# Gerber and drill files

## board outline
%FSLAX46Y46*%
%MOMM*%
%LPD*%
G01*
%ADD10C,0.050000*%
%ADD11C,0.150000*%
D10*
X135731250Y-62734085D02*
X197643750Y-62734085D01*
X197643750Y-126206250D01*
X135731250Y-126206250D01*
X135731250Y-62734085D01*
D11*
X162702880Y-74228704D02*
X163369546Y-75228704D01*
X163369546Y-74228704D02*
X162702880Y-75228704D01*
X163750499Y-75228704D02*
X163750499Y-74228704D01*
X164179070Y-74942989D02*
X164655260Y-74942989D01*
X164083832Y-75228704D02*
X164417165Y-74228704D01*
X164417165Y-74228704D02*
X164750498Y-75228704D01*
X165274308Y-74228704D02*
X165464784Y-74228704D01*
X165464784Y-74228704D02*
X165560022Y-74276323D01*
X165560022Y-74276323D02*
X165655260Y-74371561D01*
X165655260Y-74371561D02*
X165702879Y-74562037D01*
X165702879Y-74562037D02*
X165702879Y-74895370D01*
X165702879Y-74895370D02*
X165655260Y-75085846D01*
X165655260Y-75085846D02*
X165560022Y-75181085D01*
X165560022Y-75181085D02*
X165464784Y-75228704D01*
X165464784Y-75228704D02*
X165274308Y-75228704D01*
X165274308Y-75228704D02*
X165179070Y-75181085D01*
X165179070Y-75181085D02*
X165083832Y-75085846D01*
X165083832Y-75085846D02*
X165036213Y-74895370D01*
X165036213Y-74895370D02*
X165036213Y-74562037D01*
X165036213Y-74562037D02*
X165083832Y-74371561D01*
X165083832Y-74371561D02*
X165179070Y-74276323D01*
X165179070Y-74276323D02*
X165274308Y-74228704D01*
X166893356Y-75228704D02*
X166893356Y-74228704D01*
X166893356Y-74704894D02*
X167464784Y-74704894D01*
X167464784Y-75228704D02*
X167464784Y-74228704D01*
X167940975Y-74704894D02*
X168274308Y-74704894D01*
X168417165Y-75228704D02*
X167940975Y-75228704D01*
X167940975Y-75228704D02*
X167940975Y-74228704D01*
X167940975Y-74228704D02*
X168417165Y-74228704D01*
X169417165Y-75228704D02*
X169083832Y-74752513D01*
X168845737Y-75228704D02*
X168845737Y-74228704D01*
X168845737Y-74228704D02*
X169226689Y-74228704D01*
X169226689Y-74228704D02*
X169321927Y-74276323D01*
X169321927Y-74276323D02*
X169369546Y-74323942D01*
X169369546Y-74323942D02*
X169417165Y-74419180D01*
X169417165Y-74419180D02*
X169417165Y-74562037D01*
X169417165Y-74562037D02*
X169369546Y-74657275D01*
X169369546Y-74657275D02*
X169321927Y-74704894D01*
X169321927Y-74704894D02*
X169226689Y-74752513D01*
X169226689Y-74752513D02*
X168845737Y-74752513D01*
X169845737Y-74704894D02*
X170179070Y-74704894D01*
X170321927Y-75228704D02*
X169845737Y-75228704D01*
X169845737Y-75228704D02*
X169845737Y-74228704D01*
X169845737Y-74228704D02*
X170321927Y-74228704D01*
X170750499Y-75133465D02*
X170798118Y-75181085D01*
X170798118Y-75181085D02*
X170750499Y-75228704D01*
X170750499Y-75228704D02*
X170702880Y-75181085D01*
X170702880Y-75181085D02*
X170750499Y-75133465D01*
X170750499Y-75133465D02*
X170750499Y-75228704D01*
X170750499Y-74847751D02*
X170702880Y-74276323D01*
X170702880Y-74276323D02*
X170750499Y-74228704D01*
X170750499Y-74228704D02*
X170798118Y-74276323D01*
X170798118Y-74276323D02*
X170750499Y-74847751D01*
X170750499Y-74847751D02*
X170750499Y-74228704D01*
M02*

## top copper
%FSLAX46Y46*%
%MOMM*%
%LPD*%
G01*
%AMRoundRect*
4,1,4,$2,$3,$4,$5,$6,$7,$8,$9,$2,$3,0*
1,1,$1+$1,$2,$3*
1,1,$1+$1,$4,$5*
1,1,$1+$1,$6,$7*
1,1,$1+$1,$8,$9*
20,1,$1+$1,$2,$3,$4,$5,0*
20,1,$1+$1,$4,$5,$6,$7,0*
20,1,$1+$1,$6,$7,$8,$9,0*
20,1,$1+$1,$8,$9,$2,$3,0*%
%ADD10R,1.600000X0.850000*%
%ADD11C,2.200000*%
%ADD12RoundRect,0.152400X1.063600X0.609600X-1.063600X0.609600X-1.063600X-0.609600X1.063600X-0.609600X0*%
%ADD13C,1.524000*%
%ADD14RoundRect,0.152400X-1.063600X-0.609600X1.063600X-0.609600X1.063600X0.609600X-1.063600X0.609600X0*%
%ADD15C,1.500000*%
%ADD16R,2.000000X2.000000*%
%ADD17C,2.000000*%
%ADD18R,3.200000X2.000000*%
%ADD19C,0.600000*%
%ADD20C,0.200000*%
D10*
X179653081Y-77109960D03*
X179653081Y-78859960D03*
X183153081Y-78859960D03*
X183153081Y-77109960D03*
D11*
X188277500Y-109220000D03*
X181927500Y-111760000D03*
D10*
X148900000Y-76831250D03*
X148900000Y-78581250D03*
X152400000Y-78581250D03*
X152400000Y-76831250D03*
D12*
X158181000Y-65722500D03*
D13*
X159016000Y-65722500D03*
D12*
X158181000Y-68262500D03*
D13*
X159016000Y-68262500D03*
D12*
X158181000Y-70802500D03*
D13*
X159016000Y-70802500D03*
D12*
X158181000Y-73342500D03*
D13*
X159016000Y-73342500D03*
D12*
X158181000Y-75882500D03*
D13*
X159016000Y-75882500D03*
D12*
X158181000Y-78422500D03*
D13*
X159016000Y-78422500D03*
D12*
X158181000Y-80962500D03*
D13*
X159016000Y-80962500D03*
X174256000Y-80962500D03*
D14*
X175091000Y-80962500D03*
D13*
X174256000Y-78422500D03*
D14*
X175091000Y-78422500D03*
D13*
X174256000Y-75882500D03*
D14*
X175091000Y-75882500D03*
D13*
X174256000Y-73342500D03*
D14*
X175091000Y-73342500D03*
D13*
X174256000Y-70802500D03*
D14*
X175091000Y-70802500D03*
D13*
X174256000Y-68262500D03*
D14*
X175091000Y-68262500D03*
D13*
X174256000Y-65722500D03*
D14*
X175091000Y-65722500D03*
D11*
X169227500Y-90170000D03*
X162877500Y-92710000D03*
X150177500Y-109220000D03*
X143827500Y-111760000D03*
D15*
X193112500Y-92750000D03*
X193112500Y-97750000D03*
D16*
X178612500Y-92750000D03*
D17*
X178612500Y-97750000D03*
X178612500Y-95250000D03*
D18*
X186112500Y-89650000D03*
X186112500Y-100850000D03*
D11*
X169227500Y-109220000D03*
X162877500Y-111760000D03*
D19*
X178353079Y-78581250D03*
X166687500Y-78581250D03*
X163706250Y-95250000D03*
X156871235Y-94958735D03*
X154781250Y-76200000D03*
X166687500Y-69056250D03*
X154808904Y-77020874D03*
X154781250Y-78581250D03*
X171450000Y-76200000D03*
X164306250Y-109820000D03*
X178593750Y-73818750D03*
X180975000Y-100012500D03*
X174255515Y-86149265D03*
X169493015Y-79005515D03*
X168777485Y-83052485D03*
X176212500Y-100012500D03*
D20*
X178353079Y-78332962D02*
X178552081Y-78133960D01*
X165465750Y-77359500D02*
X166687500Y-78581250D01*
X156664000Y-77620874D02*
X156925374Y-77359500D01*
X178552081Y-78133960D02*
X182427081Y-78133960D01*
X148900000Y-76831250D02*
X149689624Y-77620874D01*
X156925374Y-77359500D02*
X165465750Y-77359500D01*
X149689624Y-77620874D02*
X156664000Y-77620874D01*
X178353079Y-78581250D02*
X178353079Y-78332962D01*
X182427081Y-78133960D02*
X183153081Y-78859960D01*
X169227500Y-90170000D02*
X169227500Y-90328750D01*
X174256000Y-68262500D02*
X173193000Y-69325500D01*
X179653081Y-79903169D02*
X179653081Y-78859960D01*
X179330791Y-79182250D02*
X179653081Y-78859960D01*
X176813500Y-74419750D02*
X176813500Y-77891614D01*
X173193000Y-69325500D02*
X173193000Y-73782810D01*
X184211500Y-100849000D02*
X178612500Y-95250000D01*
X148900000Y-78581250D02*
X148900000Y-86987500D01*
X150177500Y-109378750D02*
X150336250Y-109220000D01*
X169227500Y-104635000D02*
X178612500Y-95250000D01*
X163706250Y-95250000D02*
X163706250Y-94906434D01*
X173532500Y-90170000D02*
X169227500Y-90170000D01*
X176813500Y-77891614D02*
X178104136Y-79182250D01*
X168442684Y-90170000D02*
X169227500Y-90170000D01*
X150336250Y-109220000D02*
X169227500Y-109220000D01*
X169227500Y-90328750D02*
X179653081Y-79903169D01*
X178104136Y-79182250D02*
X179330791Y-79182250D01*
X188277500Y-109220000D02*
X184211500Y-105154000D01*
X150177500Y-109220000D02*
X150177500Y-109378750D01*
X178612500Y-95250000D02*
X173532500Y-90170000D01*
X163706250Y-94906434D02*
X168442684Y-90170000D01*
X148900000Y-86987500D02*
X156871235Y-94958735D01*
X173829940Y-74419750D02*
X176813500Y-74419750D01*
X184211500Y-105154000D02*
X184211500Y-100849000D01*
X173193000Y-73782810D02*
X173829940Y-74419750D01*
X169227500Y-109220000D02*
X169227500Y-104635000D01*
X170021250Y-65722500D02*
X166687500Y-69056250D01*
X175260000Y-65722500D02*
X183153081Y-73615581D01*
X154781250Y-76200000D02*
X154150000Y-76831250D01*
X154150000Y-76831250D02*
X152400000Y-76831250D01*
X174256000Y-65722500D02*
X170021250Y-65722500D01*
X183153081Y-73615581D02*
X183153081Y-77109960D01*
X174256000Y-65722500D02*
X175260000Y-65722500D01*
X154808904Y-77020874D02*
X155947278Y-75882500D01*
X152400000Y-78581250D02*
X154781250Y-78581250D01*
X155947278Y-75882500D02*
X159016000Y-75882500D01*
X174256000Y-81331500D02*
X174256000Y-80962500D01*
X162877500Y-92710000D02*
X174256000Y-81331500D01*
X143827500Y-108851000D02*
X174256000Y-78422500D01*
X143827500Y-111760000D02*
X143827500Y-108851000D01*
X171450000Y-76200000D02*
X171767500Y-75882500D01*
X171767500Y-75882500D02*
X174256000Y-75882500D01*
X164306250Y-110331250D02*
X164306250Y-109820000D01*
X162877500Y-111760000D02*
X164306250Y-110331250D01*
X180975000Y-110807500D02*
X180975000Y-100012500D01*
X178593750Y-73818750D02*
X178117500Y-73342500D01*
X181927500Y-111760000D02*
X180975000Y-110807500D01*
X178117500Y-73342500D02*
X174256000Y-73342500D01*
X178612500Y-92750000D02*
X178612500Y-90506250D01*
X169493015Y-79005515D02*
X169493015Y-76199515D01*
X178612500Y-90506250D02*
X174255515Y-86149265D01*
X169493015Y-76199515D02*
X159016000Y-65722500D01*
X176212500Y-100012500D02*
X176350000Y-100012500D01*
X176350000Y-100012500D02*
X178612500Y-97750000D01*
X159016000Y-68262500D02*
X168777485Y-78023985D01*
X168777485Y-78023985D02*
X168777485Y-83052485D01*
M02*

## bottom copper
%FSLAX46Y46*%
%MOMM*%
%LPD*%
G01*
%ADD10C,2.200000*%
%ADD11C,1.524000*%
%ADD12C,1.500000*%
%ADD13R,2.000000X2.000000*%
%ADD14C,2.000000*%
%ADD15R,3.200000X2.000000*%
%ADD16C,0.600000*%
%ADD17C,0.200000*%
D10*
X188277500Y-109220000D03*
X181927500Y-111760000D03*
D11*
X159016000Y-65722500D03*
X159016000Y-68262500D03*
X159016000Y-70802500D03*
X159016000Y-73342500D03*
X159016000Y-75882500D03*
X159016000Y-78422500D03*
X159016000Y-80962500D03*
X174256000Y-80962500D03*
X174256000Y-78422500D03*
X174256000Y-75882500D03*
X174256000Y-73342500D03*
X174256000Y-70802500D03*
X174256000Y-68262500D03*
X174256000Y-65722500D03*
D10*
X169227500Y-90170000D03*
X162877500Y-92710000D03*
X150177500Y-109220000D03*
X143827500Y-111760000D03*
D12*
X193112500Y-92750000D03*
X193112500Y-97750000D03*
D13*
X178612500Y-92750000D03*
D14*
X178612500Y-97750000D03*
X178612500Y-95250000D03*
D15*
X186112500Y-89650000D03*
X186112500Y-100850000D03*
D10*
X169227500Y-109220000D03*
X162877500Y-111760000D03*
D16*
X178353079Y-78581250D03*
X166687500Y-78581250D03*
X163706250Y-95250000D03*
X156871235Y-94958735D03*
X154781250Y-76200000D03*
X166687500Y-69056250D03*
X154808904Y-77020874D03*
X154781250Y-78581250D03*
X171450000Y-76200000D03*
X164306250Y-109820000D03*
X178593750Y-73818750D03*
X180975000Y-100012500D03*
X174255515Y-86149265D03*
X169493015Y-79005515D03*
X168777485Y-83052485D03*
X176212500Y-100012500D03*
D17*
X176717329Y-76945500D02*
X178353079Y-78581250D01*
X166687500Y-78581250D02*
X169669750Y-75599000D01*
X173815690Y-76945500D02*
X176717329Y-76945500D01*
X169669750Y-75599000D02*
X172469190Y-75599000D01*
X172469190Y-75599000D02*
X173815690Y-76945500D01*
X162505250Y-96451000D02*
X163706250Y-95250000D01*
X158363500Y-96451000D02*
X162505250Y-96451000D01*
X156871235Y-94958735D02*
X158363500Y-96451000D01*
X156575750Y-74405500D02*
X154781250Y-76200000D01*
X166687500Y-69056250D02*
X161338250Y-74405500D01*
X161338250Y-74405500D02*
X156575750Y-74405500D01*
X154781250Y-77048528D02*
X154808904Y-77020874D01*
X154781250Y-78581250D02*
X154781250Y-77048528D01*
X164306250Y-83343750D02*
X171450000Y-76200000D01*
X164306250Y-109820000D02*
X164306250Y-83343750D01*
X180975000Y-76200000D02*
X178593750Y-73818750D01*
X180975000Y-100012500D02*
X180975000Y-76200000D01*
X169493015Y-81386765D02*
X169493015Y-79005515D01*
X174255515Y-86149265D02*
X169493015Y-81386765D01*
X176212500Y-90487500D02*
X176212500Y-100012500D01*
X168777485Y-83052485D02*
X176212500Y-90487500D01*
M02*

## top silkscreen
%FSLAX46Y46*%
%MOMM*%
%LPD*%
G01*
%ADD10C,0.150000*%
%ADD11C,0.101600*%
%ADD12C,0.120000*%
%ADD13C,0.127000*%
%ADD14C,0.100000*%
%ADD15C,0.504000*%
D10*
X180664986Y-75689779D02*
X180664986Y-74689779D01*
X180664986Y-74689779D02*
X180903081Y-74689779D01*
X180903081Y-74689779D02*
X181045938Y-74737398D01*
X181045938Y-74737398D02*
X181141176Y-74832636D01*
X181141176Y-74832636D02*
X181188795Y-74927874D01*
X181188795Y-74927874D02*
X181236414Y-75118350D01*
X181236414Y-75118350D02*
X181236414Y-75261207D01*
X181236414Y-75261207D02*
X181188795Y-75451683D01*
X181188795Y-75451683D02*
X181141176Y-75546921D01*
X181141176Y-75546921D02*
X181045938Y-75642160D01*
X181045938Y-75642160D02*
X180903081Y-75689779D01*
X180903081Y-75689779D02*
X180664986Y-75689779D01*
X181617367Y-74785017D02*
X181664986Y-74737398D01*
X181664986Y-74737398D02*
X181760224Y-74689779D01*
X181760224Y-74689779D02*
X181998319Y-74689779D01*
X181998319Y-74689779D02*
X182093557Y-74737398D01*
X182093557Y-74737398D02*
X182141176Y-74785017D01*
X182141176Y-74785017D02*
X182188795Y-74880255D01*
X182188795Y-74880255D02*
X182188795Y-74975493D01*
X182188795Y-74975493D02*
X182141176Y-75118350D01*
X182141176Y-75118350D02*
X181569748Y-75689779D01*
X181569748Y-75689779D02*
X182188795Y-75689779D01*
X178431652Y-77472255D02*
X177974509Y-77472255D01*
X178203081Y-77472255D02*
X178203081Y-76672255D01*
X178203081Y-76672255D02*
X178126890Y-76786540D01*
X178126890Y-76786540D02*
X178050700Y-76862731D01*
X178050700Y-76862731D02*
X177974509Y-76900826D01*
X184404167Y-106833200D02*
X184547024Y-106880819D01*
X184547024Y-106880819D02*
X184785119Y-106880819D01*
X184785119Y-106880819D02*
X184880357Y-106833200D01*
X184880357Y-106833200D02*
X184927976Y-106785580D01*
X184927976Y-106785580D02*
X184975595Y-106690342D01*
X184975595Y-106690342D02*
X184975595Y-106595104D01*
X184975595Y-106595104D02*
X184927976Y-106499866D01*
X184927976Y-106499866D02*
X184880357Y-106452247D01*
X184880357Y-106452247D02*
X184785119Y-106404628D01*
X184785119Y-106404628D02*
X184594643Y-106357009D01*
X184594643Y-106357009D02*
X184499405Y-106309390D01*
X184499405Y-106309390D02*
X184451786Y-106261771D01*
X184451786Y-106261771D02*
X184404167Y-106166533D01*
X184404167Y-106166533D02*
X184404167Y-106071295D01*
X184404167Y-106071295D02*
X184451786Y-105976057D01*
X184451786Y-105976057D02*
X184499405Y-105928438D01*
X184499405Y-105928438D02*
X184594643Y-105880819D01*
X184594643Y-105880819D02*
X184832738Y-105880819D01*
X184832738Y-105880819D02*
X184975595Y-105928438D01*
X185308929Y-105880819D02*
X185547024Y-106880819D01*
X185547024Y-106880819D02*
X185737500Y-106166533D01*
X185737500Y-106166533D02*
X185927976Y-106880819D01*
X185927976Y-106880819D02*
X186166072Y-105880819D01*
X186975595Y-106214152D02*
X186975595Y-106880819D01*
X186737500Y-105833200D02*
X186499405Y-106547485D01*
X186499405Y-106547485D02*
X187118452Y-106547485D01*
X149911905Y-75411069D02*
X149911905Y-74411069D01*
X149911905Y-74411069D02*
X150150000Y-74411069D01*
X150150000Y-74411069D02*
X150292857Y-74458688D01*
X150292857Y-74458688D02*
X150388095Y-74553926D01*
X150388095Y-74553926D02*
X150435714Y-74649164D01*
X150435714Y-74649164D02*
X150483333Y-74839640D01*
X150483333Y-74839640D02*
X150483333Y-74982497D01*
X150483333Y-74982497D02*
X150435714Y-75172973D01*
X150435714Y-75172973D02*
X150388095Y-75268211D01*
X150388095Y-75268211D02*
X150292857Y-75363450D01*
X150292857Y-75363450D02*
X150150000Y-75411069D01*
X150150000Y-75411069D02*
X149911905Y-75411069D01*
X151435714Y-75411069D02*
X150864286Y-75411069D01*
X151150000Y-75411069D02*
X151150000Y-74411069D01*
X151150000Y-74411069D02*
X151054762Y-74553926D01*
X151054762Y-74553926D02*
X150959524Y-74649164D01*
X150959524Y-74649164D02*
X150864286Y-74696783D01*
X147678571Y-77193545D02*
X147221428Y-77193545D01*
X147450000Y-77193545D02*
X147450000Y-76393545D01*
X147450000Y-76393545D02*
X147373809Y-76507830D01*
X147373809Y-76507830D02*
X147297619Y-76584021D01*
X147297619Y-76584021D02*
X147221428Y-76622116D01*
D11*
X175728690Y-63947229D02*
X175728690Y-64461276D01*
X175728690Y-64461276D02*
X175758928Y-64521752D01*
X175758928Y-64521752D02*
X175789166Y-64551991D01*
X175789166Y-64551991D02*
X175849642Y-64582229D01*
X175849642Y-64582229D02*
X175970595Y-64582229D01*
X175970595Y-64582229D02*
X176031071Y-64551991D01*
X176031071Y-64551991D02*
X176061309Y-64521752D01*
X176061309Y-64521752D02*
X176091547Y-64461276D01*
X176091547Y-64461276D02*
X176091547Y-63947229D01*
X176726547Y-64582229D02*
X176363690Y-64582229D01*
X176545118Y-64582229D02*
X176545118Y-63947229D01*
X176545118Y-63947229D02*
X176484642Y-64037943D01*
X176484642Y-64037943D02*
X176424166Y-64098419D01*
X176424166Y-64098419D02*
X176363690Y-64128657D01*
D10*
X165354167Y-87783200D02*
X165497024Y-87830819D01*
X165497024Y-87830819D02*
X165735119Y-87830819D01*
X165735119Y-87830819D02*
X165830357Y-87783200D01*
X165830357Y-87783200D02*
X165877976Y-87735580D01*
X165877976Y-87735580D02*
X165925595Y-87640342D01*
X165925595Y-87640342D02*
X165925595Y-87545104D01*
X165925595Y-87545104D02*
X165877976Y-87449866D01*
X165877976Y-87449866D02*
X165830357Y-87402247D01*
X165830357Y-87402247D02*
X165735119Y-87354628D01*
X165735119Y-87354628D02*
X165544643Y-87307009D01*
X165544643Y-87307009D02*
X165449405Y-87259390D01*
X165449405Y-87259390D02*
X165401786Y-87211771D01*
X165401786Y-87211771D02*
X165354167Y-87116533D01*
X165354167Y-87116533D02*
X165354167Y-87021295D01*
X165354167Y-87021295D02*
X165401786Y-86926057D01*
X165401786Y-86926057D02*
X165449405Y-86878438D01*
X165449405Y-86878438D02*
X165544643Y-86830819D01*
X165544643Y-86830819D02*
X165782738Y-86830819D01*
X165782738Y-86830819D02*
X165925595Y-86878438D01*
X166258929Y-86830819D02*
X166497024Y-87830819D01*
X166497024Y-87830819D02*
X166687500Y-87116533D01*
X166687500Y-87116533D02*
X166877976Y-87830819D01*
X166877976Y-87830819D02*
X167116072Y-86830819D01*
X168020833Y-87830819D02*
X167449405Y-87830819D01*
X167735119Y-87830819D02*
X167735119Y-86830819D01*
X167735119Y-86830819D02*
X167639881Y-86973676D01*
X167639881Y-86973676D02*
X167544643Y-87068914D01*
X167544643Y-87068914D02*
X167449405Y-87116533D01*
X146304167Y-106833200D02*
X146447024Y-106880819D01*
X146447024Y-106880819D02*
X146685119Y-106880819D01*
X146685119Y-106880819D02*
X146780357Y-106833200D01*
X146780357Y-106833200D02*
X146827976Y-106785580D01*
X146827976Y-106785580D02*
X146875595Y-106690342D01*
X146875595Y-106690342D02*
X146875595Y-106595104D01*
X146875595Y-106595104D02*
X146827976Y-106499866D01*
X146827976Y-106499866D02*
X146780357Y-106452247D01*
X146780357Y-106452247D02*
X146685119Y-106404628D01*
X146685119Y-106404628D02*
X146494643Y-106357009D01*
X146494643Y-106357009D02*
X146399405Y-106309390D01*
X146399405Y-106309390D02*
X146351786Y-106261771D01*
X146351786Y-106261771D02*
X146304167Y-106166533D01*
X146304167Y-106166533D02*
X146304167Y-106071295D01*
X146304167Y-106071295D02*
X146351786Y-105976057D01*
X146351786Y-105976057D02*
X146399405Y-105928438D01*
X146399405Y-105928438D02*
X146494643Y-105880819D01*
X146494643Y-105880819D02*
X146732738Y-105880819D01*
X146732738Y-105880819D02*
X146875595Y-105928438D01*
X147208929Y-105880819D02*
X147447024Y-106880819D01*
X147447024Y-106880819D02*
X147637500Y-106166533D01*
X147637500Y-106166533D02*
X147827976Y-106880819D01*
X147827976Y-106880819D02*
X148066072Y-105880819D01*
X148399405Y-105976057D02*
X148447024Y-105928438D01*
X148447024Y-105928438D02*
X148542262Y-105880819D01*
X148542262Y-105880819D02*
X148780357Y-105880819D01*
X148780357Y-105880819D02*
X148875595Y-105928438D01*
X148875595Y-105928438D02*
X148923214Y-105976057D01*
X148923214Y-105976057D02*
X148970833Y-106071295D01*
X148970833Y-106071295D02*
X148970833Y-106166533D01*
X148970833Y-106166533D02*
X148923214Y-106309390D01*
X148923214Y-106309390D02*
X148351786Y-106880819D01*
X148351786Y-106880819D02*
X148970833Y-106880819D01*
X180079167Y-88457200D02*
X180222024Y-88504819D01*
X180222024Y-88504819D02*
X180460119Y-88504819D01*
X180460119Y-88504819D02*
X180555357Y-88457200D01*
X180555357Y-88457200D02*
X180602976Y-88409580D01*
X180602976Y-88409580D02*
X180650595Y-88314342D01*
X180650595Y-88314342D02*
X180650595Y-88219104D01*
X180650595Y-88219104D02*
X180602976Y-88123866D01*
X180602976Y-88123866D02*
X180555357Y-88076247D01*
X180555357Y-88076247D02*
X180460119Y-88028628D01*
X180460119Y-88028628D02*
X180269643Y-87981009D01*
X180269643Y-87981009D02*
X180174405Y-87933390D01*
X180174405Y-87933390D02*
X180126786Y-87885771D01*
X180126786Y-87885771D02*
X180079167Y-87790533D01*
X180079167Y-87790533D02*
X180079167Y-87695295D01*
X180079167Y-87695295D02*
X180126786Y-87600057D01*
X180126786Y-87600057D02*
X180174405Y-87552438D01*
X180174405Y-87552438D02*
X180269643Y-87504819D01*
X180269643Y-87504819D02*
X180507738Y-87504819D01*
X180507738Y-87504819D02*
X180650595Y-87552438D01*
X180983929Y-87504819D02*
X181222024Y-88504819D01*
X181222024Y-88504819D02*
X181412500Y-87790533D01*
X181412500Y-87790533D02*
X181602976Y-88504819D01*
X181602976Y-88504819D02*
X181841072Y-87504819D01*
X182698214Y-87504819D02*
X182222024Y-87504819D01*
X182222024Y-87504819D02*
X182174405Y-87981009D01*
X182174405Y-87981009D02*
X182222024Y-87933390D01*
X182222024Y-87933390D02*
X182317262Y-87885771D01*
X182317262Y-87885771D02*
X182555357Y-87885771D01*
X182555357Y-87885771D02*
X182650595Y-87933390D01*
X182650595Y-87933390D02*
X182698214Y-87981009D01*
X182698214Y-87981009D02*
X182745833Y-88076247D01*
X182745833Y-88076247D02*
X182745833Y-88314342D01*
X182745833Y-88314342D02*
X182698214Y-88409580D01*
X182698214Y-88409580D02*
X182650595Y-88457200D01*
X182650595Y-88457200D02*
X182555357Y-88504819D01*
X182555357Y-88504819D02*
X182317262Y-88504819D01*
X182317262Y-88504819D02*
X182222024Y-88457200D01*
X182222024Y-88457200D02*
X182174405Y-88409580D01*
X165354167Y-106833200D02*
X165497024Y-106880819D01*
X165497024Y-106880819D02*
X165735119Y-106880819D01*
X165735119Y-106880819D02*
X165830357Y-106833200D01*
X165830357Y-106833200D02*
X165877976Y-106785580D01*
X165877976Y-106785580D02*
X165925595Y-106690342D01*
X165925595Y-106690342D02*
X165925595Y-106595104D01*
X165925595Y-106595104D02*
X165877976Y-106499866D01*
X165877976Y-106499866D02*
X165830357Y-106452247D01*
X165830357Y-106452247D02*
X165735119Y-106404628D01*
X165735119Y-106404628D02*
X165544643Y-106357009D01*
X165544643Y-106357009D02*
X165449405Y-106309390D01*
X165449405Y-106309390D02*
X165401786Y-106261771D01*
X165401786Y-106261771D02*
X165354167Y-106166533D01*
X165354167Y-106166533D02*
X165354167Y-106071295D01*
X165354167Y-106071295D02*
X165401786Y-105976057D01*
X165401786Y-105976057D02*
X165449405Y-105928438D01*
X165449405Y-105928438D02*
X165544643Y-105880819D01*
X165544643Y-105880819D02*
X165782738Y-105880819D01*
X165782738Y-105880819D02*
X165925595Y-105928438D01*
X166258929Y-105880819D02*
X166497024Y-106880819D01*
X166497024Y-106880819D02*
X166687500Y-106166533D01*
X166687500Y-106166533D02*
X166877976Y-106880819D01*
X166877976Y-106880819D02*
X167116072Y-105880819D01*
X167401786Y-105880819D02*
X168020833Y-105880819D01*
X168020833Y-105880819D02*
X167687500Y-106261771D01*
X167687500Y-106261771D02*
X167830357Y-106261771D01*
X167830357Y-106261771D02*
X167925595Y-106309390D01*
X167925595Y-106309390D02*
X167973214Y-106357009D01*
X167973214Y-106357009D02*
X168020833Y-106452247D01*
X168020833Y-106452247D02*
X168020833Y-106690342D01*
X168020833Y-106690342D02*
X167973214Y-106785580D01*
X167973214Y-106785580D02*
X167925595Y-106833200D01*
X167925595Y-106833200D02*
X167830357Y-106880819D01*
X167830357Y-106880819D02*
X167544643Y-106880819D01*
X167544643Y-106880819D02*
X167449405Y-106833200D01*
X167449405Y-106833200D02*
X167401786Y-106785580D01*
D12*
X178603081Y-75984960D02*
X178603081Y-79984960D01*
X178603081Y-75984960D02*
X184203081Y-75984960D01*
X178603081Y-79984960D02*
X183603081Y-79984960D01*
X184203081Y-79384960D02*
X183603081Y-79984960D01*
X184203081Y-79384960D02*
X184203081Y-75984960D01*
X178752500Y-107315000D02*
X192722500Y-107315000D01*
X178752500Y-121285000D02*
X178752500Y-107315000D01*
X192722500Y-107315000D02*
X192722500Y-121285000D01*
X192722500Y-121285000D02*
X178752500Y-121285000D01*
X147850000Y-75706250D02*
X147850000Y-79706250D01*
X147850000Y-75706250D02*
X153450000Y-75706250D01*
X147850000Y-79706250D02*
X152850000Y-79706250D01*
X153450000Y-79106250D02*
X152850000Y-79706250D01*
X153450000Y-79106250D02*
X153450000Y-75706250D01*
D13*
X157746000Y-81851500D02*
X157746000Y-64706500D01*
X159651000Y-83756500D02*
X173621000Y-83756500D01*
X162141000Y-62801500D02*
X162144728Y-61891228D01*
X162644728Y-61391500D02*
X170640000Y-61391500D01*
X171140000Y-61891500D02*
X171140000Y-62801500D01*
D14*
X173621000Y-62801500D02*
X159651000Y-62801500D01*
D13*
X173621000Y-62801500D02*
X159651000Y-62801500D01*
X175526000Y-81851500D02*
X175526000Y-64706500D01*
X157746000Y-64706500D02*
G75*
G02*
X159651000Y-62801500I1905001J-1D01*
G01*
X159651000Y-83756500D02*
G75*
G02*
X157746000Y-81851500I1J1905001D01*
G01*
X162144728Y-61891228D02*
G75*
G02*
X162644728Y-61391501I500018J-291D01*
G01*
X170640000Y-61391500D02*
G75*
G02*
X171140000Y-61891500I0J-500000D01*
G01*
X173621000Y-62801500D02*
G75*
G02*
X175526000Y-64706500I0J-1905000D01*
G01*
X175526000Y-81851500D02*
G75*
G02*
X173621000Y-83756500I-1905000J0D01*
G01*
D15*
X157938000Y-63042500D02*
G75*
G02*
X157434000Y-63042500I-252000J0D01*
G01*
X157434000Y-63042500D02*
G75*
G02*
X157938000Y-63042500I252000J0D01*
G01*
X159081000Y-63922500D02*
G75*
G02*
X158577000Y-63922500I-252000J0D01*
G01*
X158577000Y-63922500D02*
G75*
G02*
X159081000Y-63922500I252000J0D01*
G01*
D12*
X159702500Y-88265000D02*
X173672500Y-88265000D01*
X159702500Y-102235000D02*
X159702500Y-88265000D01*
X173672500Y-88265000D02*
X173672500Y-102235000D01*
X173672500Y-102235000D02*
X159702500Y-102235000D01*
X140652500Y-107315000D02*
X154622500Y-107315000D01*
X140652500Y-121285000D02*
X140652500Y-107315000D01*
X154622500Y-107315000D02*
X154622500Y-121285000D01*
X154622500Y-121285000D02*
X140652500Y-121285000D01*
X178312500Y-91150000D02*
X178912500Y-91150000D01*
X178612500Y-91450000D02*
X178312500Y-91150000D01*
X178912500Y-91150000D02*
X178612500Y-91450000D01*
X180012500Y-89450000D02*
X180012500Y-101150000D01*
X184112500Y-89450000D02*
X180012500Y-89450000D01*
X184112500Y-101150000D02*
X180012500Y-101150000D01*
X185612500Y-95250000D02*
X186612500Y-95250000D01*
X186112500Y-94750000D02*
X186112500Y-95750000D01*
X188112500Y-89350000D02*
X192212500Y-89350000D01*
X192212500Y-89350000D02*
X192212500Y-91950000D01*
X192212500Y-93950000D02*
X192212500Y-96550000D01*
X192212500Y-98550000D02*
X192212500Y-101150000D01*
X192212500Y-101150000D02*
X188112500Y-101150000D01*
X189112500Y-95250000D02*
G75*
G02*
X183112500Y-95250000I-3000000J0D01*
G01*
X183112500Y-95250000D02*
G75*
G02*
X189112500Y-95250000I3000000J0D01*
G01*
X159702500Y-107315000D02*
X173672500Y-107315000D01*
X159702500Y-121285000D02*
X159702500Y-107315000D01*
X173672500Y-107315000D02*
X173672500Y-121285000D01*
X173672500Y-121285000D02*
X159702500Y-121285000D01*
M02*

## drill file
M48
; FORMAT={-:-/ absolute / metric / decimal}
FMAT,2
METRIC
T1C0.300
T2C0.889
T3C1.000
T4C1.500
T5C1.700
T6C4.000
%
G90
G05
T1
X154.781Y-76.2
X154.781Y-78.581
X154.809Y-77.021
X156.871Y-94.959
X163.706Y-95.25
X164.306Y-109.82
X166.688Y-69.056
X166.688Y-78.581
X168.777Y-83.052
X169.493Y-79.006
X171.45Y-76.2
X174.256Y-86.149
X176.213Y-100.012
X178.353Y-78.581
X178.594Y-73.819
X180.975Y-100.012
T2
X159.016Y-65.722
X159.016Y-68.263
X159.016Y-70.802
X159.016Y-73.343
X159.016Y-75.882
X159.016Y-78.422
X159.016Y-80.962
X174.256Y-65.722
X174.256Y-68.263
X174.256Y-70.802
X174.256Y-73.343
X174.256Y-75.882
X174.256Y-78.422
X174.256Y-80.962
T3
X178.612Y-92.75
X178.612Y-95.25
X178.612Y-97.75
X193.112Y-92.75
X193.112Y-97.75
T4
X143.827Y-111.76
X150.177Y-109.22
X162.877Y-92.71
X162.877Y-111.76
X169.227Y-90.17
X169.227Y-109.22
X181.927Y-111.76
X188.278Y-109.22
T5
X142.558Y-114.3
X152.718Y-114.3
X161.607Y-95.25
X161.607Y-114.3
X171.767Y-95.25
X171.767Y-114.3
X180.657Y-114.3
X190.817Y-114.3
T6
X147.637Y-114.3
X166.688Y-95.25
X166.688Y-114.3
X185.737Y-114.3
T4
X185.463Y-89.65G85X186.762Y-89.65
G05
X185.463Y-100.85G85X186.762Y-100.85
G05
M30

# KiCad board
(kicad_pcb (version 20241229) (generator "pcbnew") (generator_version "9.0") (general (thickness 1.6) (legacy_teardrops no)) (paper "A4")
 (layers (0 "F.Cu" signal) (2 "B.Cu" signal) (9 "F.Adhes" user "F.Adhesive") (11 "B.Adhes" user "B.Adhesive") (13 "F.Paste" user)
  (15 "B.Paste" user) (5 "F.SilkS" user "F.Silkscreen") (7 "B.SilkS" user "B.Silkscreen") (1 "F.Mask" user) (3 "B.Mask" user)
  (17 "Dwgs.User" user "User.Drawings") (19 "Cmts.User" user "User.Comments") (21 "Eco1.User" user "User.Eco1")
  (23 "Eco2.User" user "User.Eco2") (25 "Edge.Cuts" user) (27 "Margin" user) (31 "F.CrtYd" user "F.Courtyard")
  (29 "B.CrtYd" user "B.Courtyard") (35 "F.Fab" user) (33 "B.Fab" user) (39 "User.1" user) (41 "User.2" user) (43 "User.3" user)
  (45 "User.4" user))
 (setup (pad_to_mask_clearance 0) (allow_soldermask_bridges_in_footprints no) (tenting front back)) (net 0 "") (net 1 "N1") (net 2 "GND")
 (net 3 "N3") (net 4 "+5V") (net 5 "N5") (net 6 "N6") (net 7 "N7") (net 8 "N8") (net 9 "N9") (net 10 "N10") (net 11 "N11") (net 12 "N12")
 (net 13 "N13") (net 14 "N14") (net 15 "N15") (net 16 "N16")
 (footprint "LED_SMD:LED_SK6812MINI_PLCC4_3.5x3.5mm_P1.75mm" (layer "F.Cu") (at 181.403081 77.98496)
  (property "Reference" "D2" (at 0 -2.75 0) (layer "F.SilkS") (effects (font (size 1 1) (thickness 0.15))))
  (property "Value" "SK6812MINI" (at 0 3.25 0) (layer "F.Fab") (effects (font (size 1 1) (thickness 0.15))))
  (fp_line (start -2.8 -2) (end -2.8 2) (stroke (width 0.12) (type default)) (layer "F.SilkS"))
  (fp_line (start -2.8 -2) (end 2.8 -2) (stroke (width 0.12) (type solid)) (layer "F.SilkS"))
  (fp_line (start -2.8 2) (end 2.2 2) (stroke (width 0.12) (type solid)) (layer "F.SilkS"))
  (fp_line (start 2.8 1.4) (end 2.2 2) (stroke (width 0.12) (type default)) (layer "F.SilkS"))
  (fp_line (start 2.8 1.4) (end 2.8 -2) (stroke (width 0.12) (type solid)) (layer "F.SilkS"))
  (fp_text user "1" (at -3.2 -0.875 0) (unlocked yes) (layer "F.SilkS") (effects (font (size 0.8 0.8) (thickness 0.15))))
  (pad "1" smd rect (at -1.75 -0.875) (size 1.6 0.85) (layers "F.Cu" "F.Mask" "F.Paste") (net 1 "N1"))
  (pad "2" smd rect (at -1.75 0.875) (size 1.6 0.85) (layers "F.Cu" "F.Mask" "F.Paste") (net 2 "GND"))
  (pad "3" smd rect (at 1.75 0.875) (size 1.6 0.85) (layers "F.Cu" "F.Mask" "F.Paste") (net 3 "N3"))
  (pad "4" smd rect (at 1.75 -0.875) (size 1.6 0.85) (layers "F.Cu" "F.Mask" "F.Paste") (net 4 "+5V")))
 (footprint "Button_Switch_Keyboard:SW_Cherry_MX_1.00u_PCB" (layer "F.Cu") (at 188.2775 109.22)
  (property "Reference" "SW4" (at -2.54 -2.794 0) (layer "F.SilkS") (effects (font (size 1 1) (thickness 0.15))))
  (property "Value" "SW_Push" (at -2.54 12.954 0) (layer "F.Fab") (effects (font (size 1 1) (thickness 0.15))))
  (fp_line (start -9.525 -1.905) (end 4.445 -1.905) (stroke (width 0.12) (type solid)) (layer "F.SilkS"))
  (fp_line (start -9.525 12.065) (end -9.525 -1.905) (stroke (width 0.12) (type solid)) (layer "F.SilkS"))
  (fp_line (start 4.445 -1.905) (end 4.445 12.065) (stroke (width 0.12) (type solid)) (layer "F.SilkS"))
  (fp_line (start 4.445 12.065) (end -9.525 12.065) (stroke (width 0.12) (type solid)) (layer "F.SilkS"))
  (pad "" np_thru_hole circle (at -7.62 5.08) (size 1.7 1.7) (drill 1.7) (layers "*.Cu" "*.Mask"))
  (pad "" np_thru_hole circle (at -2.54 5.08) (size 4 4) (drill 4) (layers "*.Cu" "*.Mask"))
  (pad "" np_thru_hole circle (at 2.54 5.08) (size 1.7 1.7) (drill 1.7) (layers "*.Cu" "*.Mask"))
  (pad "1" thru_hole circle (at 0 0) (size 2.2 2.2) (drill 1.5) (layers "*.Cu" "*.Mask") (remove_unused_layers no) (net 2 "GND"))
  (pad "2" thru_hole circle (at -6.35 2.54) (size 2.2 2.2) (drill 1.5) (layers "*.Cu" "*.Mask") (remove_unused_layers no) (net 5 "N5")))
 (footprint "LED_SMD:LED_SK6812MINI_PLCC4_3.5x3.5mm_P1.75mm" (layer "F.Cu") (at 150.65 77.70625)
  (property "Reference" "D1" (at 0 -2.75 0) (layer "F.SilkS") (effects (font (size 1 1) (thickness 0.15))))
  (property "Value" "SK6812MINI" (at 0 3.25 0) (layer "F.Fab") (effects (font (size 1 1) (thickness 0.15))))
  (fp_line (start -2.8 -2) (end -2.8 2) (stroke (width 0.12) (type default)) (layer "F.SilkS"))
  (fp_line (start -2.8 -2) (end 2.8 -2) (stroke (width 0.12) (type solid)) (layer "F.SilkS"))
  (fp_line (start -2.8 2) (end 2.2 2) (stroke (width 0.12) (type solid)) (layer "F.SilkS"))
  (fp_line (start 2.8 1.4) (end 2.2 2) (stroke (width 0.12) (type default)) (layer "F.SilkS"))
  (fp_line (start 2.8 1.4) (end 2.8 -2) (stroke (width 0.12) (type solid)) (layer "F.SilkS"))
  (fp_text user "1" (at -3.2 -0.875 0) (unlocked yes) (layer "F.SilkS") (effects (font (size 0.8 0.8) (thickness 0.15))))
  (pad "1" smd rect (at -1.75 -0.875) (size 1.6 0.85) (layers "F.Cu" "F.Mask" "F.Paste") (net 3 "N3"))
  (pad "2" smd rect (at -1.75 0.875) (size 1.6 0.85) (layers "F.Cu" "F.Mask" "F.Paste") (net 2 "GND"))
  (pad "3" smd rect (at 1.75 0.875) (size 1.6 0.85) (layers "F.Cu" "F.Mask" "F.Paste") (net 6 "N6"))
  (pad "4" smd rect (at 1.75 -0.875) (size 1.6 0.85) (layers "F.Cu" "F.Mask" "F.Paste") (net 4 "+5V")))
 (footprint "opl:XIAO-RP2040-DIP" (layer "F.Cu") (at 166.636 73.3425)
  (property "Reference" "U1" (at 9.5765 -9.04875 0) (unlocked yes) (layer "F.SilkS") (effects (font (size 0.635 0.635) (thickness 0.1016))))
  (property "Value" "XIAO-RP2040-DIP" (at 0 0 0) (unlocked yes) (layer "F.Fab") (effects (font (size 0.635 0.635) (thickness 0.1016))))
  (fp_line (start -8.89 8.509) (end -8.89 -8.636) (stroke (width 0.127) (type solid)) (layer "F.SilkS"))
  (fp_line (start -6.985 10.414) (end 6.985 10.414) (stroke (width 0.127) (type solid)) (layer "F.SilkS"))
  (fp_line (start -4.495 -10.541) (end -4.491272 -11.451272) (stroke (width 0.127) (type solid)) (layer "F.SilkS"))
  (fp_line (start -3.991272 -11.951) (end 4.004 -11.951) (stroke (width 0.127) (type solid)) (layer "F.SilkS"))
  (fp_line (start 4.504 -11.451) (end 4.504 -10.541) (stroke (width 0.127) (type solid)) (layer "F.SilkS"))
  (fp_line (start 6.985 -10.541) (end -6.985 -10.541) (stroke (width 0.1) (type solid)) (layer "F.SilkS"))
  (fp_line (start 6.985 -10.541) (end -6.985 -10.541) (stroke (width 0.127) (type solid)) (layer "F.SilkS"))
  (fp_line (start 8.89 8.509) (end 8.89 -8.636) (stroke (width 0.127) (type solid)) (layer "F.SilkS"))
  (fp_arc (start -8.89 -8.636) (mid -8.332038 -9.983038) (end -6.985 -10.541) (stroke (width 0.127) (type solid)) (layer "F.SilkS"))
  (fp_arc (start -6.985 10.414) (mid -8.332038 9.856038) (end -8.89 8.509) (stroke (width 0.127) (type solid)) (layer "F.SilkS"))
  (fp_arc (start -4.491272 -11.451272) (mid -4.344728 -11.80464) (end -3.991272 -11.951) (stroke (width 0.127) (type default))
   (layer "F.SilkS"))
  (fp_arc (start 4.004 -11.951) (mid 4.357553 -11.804553) (end 4.504 -11.451) (stroke (width 0.127) (type default)) (layer "F.SilkS"))
  (fp_arc (start 6.985 -10.541) (mid 8.332038 -9.983038) (end 8.89 -8.636) (stroke (width 0.127) (type solid)) (layer "F.SilkS"))
  (fp_arc (start 8.89 8.509) (mid 8.332038 9.856038) (end 6.985 10.414) (stroke (width 0.127) (type solid)) (layer "F.SilkS"))
  (fp_circle (center -8.95 -10.3) (end -8.95 -10.554) (stroke (width 0.5) (type solid)) (fill yes) (layer "F.SilkS"))
  (fp_circle (center -7.807 -9.42) (end -7.807 -9.674) (stroke (width 0.5) (type solid)) (fill yes) (layer "F.SilkS"))
  (pad "1" smd roundrect (at -8.455 -7.62 180) (size 2.432 1.524) (layers "F.Cu" "F.Mask") (roundrect_rratio 0.1) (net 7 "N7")
   (thermal_bridge_angle 45))
  (pad "1" thru_hole circle (at -7.62 -7.62 180) (size 1.524 1.524) (drill 0.889) (layers "*.Cu" "*.Mask") (remove_unused_layers no)
   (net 7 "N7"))
  (pad "2" smd roundrect (at -8.455 -5.08 180) (size 2.432 1.524) (layers "F.Cu" "F.Mask") (roundrect_rratio 0.1) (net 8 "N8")
   (thermal_bridge_angle 45))
  (pad "2" thru_hole circle (at -7.62 -5.08 180) (size 1.524 1.524) (drill 0.889) (layers "*.Cu" "*.Mask") (remove_unused_layers no)
   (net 8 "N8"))
  (pad "3" smd roundrect (at -8.455 -2.54 180) (size 2.432 1.524) (layers "F.Cu" "F.Mask") (roundrect_rratio 0.1) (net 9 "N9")
   (thermal_bridge_angle 45))
  (pad "3" thru_hole circle (at -7.62 -2.54 180) (size 1.524 1.524) (drill 0.889) (layers "*.Cu" "*.Mask") (remove_unused_layers no)
   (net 9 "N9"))
  (pad "4" smd roundrect (at -8.455 0 180) (size 2.432 1.524) (layers "F.Cu" "F.Mask") (roundrect_rratio 0.1) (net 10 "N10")
   (thermal_bridge_angle 45))
  (pad "4" thru_hole circle (at -7.62 0 180) (size 1.524 1.524) (drill 0.889) (layers "*.Cu" "*.Mask") (remove_unused_layers no)
   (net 10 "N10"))
  (pad "5" smd roundrect (at -8.455 2.54 180) (size 2.432 1.524) (layers "F.Cu" "F.Mask") (roundrect_rratio 0.1) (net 6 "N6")
   (thermal_bridge_angle 45))
  (pad "5" thru_hole circle (at -7.62 2.54 180) (size 1.524 1.524) (drill 0.889) (layers "*.Cu" "*.Mask") (remove_unused_layers no)
   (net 6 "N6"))
  (pad "6" smd roundrect (at -8.455 5.08 180) (size 2.432 1.524) (layers "F.Cu" "F.Mask") (roundrect_rratio 0.1) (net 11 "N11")
   (thermal_bridge_angle 45))
  (pad "6" thru_hole circle (at -7.62 5.08 180) (size 1.524 1.524) (drill 0.889) (layers "*.Cu" "*.Mask") (remove_unused_layers no)
   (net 11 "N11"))
  (pad "7" smd roundrect (at -8.455 7.62 180) (size 2.432 1.524) (layers "F.Cu" "F.Mask") (roundrect_rratio 0.1) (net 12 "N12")
   (thermal_bridge_angle 45))
  (pad "7" thru_hole circle (at -7.62 7.62 180) (size 1.524 1.524) (drill 0.889) (layers "*.Cu" "*.Mask") (remove_unused_layers no)
   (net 12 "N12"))
  (pad "8" thru_hole circle (at 7.62 7.62) (size 1.524 1.524) (drill 0.889) (layers "*.Cu" "*.Mask") (remove_unused_layers no)
   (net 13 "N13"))
  (pad "8" smd roundrect (at 8.455 7.62) (size 2.432 1.524) (layers "F.Cu" "F.Mask") (roundrect_rratio 0.1) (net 13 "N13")
   (thermal_bridge_angle 45))
  (pad "9" thru_hole circle (at 7.62 5.08) (size 1.524 1.524) (drill 0.889) (layers "*.Cu" "*.Mask") (remove_unused_layers no)
   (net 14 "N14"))
  (pad "9" smd roundrect (at 8.455 5.08) (size 2.432 1.524) (layers "F.Cu" "F.Mask") (roundrect_rratio 0.1) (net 14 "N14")
   (thermal_bridge_angle 45))
  (pad "10" thru_hole circle (at 7.62 2.54) (size 1.524 1.524) (drill 0.889) (layers "*.Cu" "*.Mask") (remove_unused_layers no)
   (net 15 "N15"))
  (pad "10" smd roundrect (at 8.455 2.54) (size 2.432 1.524) (layers "F.Cu" "F.Mask") (roundrect_rratio 0.1) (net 15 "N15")
   (thermal_bridge_angle 45))
  (pad "11" thru_hole circle (at 7.62 0) (size 1.524 1.524) (drill 0.889) (layers "*.Cu" "*.Mask") (remove_unused_layers no) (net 5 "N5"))
  (pad "11" smd roundrect (at 8.455 0) (size 2.432 1.524) (layers "F.Cu" "F.Mask") (roundrect_rratio 0.1) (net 5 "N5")
   (thermal_bridge_angle 45))
  (pad "12" thru_hole circle (at 7.62 -2.54) (size 1.524 1.524) (drill 0.889) (layers "*.Cu" "*.Mask") (remove_unused_layers no)
   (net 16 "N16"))
  (pad "12" smd roundrect (at 8.455 -2.54) (size 2.432 1.524) (layers "F.Cu" "F.Mask") (roundrect_rratio 0.1) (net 16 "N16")
   (thermal_bridge_angle 45))
  (pad "13" thru_hole circle (at 7.62 -5.08) (size 1.524 1.524) (drill 0.889) (layers "*.Cu" "*.Mask") (remove_unused_layers no)
   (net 2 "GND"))
  (pad "13" smd roundrect (at 8.455 -5.08) (size 2.432 1.524) (layers "F.Cu" "F.Mask") (roundrect_rratio 0.1) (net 2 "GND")
   (thermal_bridge_angle 45))
  (pad "14" thru_hole circle (at 7.62 -7.62) (size 1.524 1.524) (drill 0.889) (layers "*.Cu" "*.Mask") (remove_unused_layers no)
   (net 4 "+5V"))
  (pad "14" smd roundrect (at 8.455 -7.62) (size 2.432 1.524) (layers "F.Cu" "F.Mask") (roundrect_rratio 0.1) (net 4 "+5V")
   (thermal_bridge_angle 45)))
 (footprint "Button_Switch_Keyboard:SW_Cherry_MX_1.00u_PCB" (layer "F.Cu") (at 169.2275 90.17)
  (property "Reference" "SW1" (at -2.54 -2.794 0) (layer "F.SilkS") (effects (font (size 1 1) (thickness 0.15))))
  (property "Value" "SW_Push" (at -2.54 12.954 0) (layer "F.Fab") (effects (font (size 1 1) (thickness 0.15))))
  (fp_line (start -9.525 -1.905) (end 4.445 -1.905) (stroke (width 0.12) (type solid)) (layer "F.SilkS"))
  (fp_line (start -9.525 12.065) (end -9.525 -1.905) (stroke (width 0.12) (type solid)) (layer "F.SilkS"))
  (fp_line (start 4.445 -1.905) (end 4.445 12.065) (stroke (width 0.12) (type solid)) (layer "F.SilkS"))
  (fp_line (start 4.445 12.065) (end -9.525 12.065) (stroke (width 0.12) (type solid)) (layer "F.SilkS"))
  (pad "" np_thru_hole circle (at -7.62 5.08) (size 1.7 1.7) (drill 1.7) (layers "*.Cu" "*.Mask"))
  (pad "" np_thru_hole circle (at -2.54 5.08) (size 4 4) (drill 4) (layers "*.Cu" "*.Mask"))
  (pad "" np_thru_hole circle (at 2.54 5.08) (size 1.7 1.7) (drill 1.7) (layers "*.Cu" "*.Mask"))
  (pad "1" thru_hole circle (at 0 0) (size 2.2 2.2) (drill 1.5) (layers "*.Cu" "*.Mask") (remove_unused_layers no) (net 2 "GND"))
  (pad "2" thru_hole circle (at -6.35 2.54) (size 2.2 2.2) (drill 1.5) (layers "*.Cu" "*.Mask") (remove_unused_layers no) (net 13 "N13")))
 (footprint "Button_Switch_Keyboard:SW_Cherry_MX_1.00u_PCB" (layer "F.Cu") (at 150.1775 109.22)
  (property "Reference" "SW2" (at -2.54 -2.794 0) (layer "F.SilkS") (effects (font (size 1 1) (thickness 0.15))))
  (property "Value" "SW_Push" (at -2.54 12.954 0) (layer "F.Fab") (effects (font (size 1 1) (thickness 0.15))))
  (fp_line (start -9.525 -1.905) (end 4.445 -1.905) (stroke (width 0.12) (type solid)) (layer "F.SilkS"))
  (fp_line (start -9.525 12.065) (end -9.525 -1.905) (stroke (width 0.12) (type solid)) (layer "F.SilkS"))
  (fp_line (start 4.445 -1.905) (end 4.445 12.065) (stroke (width 0.12) (type solid)) (layer "F.SilkS"))
  (fp_line (start 4.445 12.065) (end -9.525 12.065) (stroke (width 0.12) (type solid)) (layer "F.SilkS"))
  (pad "" np_thru_hole circle (at -7.62 5.08) (size 1.7 1.7) (drill 1.7) (layers "*.Cu" "*.Mask"))
  (pad "" np_thru_hole circle (at -2.54 5.08) (size 4 4) (drill 4) (layers "*.Cu" "*.Mask"))
  (pad "" np_thru_hole circle (at 2.54 5.08) (size 1.7 1.7) (drill 1.7) (layers "*.Cu" "*.Mask"))
  (pad "1" thru_hole circle (at 0 0) (size 2.2 2.2) (drill 1.5) (layers "*.Cu" "*.Mask") (remove_unused_layers no) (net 2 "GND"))
  (pad "2" thru_hole circle (at -6.35 2.54) (size 2.2 2.2) (drill 1.5) (layers "*.Cu" "*.Mask") (remove_unused_layers no) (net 14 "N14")))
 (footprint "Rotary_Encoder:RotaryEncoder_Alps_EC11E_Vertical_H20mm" (layer "F.Cu") (at 178.6125 92.75)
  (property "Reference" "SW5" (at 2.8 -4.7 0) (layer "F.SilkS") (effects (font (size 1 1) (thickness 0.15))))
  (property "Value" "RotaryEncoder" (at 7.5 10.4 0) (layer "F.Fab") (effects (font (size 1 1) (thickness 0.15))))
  (fp_line (start -0.3 -1.6) (end 0.3 -1.6) (stroke (width 0.12) (type solid)) (layer "F.SilkS"))
  (fp_line (start 0 -1.3) (end -0.3 -1.6) (stroke (width 0.12) (type solid)) (layer "F.SilkS"))
  (fp_line (start 0.3 -1.6) (end 0 -1.3) (stroke (width 0.12) (type solid)) (layer "F.SilkS"))
  (fp_line (start 1.4 -3.3) (end 1.4 8.4) (stroke (width 0.12) (type solid)) (layer "F.SilkS"))
  (fp_line (start 5.5 -3.3) (end 1.4 -3.3) (stroke (width 0.12) (type solid)) (layer "F.SilkS"))
  (fp_line (start 5.5 8.4) (end 1.4 8.4) (stroke (width 0.12) (type solid)) (layer "F.SilkS"))
  (fp_line (start 7 2.5) (end 8 2.5) (stroke (width 0.12) (type solid)) (layer "F.SilkS"))
  (fp_line (start 7.5 2) (end 7.5 3) (stroke (width 0.12) (type solid)) (layer "F.SilkS"))
  (fp_line (start 9.5 -3.4) (end 13.6 -3.4) (stroke (width 0.12) (type solid)) (layer "F.SilkS"))
  (fp_line (start 13.6 -3.4) (end 13.6 -0.8) (stroke (width 0.12) (type solid)) (layer "F.SilkS"))
  (fp_line (start 13.6 1.2) (end 13.6 3.8) (stroke (width 0.12) (type solid)) (layer "F.SilkS"))
  (fp_line (start 13.6 5.8) (end 13.6 8.4) (stroke (width 0.12) (type solid)) (layer "F.SilkS"))
  (fp_line (start 13.6 8.4) (end 9.5 8.4) (stroke (width 0.12) (type solid)) (layer "F.SilkS"))
  (fp_circle (center 7.5 2.5) (end 10.5 2.5) (stroke (width 0.12) (type solid)) (fill no) (layer "F.SilkS"))
  (pad "" thru_hole circle (at 14.5 0) (size 1.5 1.5) (drill 1) (layers "*.Cu" "*.Mask") (remove_unused_layers no))
  (pad "" thru_hole circle (at 14.5 5) (size 1.5 1.5) (drill 1) (layers "*.Cu" "*.Mask") (remove_unused_layers no))
  (pad "A" thru_hole rect (at 0 0) (size 2 2) (drill 1) (layers "*.Cu" "*.Mask") (remove_unused_layers no) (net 7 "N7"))
  (pad "B" thru_hole circle (at 0 5) (size 2 2) (drill 1) (layers "*.Cu" "*.Mask") (remove_unused_layers no) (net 8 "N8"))
  (pad "C" thru_hole circle (at 0 2.5) (size 2 2) (drill 1) (layers "*.Cu" "*.Mask") (remove_unused_layers no) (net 2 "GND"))
  (pad "MP" thru_hole rect (at 7.5 -3.1) (size 3.2 2) (drill oval 2.8 1.5) (layers "*.Cu" "*.Mask") (remove_unused_layers no))
  (pad "MP" thru_hole rect (at 7.5 8.1) (size 3.2 2) (drill oval 2.8 1.5) (layers "*.Cu" "*.Mask") (remove_unused_layers no)))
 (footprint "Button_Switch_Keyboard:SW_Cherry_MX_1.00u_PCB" (layer "F.Cu") (at 169.2275 109.22)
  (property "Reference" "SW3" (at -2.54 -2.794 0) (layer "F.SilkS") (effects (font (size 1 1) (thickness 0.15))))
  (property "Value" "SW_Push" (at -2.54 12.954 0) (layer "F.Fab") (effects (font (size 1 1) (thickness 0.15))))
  (fp_line (start -9.525 -1.905) (end 4.445 -1.905) (stroke (width 0.12) (type solid)) (layer "F.SilkS"))
  (fp_line (start -9.525 12.065) (end -9.525 -1.905) (stroke (width 0.12) (type solid)) (layer "F.SilkS"))
  (fp_line (start 4.445 -1.905) (end 4.445 12.065) (stroke (width 0.12) (type solid)) (layer "F.SilkS"))
  (fp_line (start 4.445 12.065) (end -9.525 12.065) (stroke (width 0.12) (type solid)) (layer "F.SilkS"))
  (pad "" np_thru_hole circle (at -7.62 5.08) (size 1.7 1.7) (drill 1.7) (layers "*.Cu" "*.Mask"))
  (pad "" np_thru_hole circle (at -2.54 5.08) (size 4 4) (drill 4) (layers "*.Cu" "*.Mask"))
  (pad "" np_thru_hole circle (at 2.54 5.08) (size 1.7 1.7) (drill 1.7) (layers "*.Cu" "*.Mask"))
  (pad "1" thru_hole circle (at 0 0) (size 2.2 2.2) (drill 1.5) (layers "*.Cu" "*.Mask") (remove_unused_layers no) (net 2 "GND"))
  (pad "2" thru_hole circle (at -6.35 2.54) (size 2.2 2.2) (drill 1.5) (layers "*.Cu" "*.Mask") (remove_unused_layers no) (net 15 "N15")))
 (gr_rect (start 135.73125 62.734085) (end 197.64375 126.20625) (stroke (width 0.05) (type default)) (fill no) (layer "Edge.Cuts"))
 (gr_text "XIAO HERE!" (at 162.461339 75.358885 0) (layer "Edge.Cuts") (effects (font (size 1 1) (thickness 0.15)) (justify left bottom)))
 (segment (start 178.353079 78.332962) (end 178.552081 78.13396) (width 0.2) (layer "F.Cu") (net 3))
 (segment (start 165.46575 77.3595) (end 166.6875 78.58125) (width 0.2) (layer "F.Cu") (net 3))
 (segment (start 156.664 77.620874) (end 156.925374 77.3595) (width 0.2) (layer "F.Cu") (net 3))
 (segment (start 178.552081 78.13396) (end 182.427081 78.13396) (width 0.2) (layer "F.Cu") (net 3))
 (segment (start 148.9 76.83125) (end 149.689624 77.620874) (width 0.2) (layer "F.Cu") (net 3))
 (segment (start 156.925374 77.3595) (end 165.46575 77.3595) (width 0.2) (layer "F.Cu") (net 3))
 (segment (start 149.689624 77.620874) (end 156.664 77.620874) (width 0.2) (layer "F.Cu") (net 3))
 (segment (start 178.353079 78.58125) (end 178.353079 78.332962) (width 0.2) (layer "F.Cu") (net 3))
 (segment (start 182.427081 78.13396) (end 183.153081 78.85996) (width 0.2) (layer "F.Cu") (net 3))
 (via (at 178.353079 78.58125) (size 0.6) (drill 0.3) (layers "F.Cu" "B.Cu") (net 3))
 (via (at 166.6875 78.58125) (size 0.6) (drill 0.3) (layers "F.Cu" "B.Cu") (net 3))
 (segment (start 176.717329 76.9455) (end 178.353079 78.58125) (width 0.2) (layer "B.Cu") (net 3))
 (segment (start 166.6875 78.58125) (end 169.66975 75.599) (width 0.2) (layer "B.Cu") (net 3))
 (segment (start 173.81569 76.9455) (end 176.717329 76.9455) (width 0.2) (layer "B.Cu") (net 3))
 (segment (start 169.66975 75.599) (end 172.46919 75.599) (width 0.2) (layer "B.Cu") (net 3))
 (segment (start 172.46919 75.599) (end 173.81569 76.9455) (width 0.2) (layer "B.Cu") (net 3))
 (segment (start 169.2275 90.17) (end 169.2275 90.32875) (width 0.2) (layer "F.Cu") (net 2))
 (segment (start 174.256 68.2625) (end 173.193 69.3255) (width 0.2) (layer "F.Cu") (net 2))
 (segment (start 179.653081 79.903169) (end 179.653081 78.85996) (width 0.2) (layer "F.Cu") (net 2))
 (segment (start 179.330791 79.18225) (end 179.653081 78.85996) (width 0.2) (layer "F.Cu") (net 2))
 (segment (start 176.8135 74.41975) (end 176.8135 77.891614) (width 0.2) (layer "F.Cu") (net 2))
 (segment (start 173.193 69.3255) (end 173.193 73.78281) (width 0.2) (layer "F.Cu") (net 2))
 (segment (start 184.2115 100.849) (end 178.6125 95.25) (width 0.2) (layer "F.Cu") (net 2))
 (segment (start 148.9 78.58125) (end 148.9 86.9875) (width 0.2) (layer "F.Cu") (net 2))
 (segment (start 150.1775 109.37875) (end 150.33625 109.22) (width 0.2) (layer "F.Cu") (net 2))
 (segment (start 169.2275 104.635) (end 178.6125 95.25) (width 0.2) (layer "F.Cu") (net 2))
 (segment (start 163.70625 95.25) (end 163.70625 94.906434) (width 0.2) (layer "F.Cu") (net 2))
 (segment (start 173.5325 90.17) (end 169.2275 90.17) (width 0.2) (layer "F.Cu") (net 2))
 (segment (start 176.8135 77.891614) (end 178.104136 79.18225) (width 0.2) (layer "F.Cu") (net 2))
 (segment (start 168.442684 90.17) (end 169.2275 90.17) (width 0.2) (layer "F.Cu") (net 2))
 (segment (start 150.33625 109.22) (end 169.2275 109.22) (width 0.2) (layer "F.Cu") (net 2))
 (segment (start 169.2275 90.32875) (end 179.653081 79.903169) (width 0.2) (layer "F.Cu") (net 2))
 (segment (start 178.104136 79.18225) (end 179.330791 79.18225) (width 0.2) (layer "F.Cu") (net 2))
 (segment (start 188.2775 109.22) (end 184.2115 105.154) (width 0.2) (layer "F.Cu") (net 2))
 (segment (start 150.1775 109.22) (end 150.1775 109.37875) (width 0.2) (layer "F.Cu") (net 2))
 (segment (start 178.6125 95.25) (end 173.5325 90.17) (width 0.2) (layer "F.Cu") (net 2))
 (segment (start 163.70625 94.906434) (end 168.442684 90.17) (width 0.2) (layer "F.Cu") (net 2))
 (segment (start 148.9 86.9875) (end 156.871235 94.958735) (width 0.2) (layer "F.Cu") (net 2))
 (segment (start 173.82994 74.41975) (end 176.8135 74.41975) (width 0.2) (layer "F.Cu") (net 2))
 (segment (start 184.2115 105.154) (end 184.2115 100.849) (width 0.2) (layer "F.Cu") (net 2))
 (segment (start 173.193 73.78281) (end 173.82994 74.41975) (width 0.2) (layer "F.Cu") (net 2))
 (segment (start 169.2275 109.22) (end 169.2275 104.635) (width 0.2) (layer "F.Cu") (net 2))
 (via (at 163.70625 95.25) (size 0.6) (drill 0.3) (layers "F.Cu" "B.Cu") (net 2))
 (via (at 156.871235 94.958735) (size 0.6) (drill 0.3) (layers "F.Cu" "B.Cu") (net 2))
 (segment (start 162.50525 96.451) (end 163.70625 95.25) (width 0.2) (layer "B.Cu") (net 2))
 (segment (start 158.3635 96.451) (end 162.50525 96.451) (width 0.2) (layer "B.Cu") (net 2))
 (segment (start 156.871235 94.958735) (end 158.3635 96.451) (width 0.2) (layer "B.Cu") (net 2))
 (segment (start 170.02125 65.7225) (end 166.6875 69.05625) (width 0.2) (layer "F.Cu") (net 4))
 (segment (start 175.26 65.7225) (end 183.153081 73.615581) (width 0.2) (layer "F.Cu") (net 4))
 (segment (start 154.78125 76.2) (end 154.15 76.83125) (width 0.2) (layer "F.Cu") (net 4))
 (segment (start 154.15 76.83125) (end 152.4 76.83125) (width 0.2) (layer "F.Cu") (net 4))
 (segment (start 174.256 65.7225) (end 170.02125 65.7225) (width 0.2) (layer "F.Cu") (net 4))
 (segment (start 183.153081 73.615581) (end 183.153081 77.10996) (width 0.2) (layer "F.Cu") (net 4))
 (segment (start 174.256 65.7225) (end 175.26 65.7225) (width 0.2) (layer "F.Cu") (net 4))
 (via (at 154.78125 76.2) (size 0.6) (drill 0.3) (layers "F.Cu" "B.Cu") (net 4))
 (via (at 166.6875 69.05625) (size 0.6) (drill 0.3) (layers "F.Cu" "B.Cu") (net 4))
 (segment (start 156.57575 74.4055) (end 154.78125 76.2) (width 0.2) (layer "B.Cu") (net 4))
 (segment (start 166.6875 69.05625) (end 161.33825 74.4055) (width 0.2) (layer "B.Cu") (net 4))
 (segment (start 161.33825 74.4055) (end 156.57575 74.4055) (width 0.2) (layer "B.Cu") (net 4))
 (segment (start 154.808904 77.020874) (end 155.947278 75.8825) (width 0.2) (layer "F.Cu") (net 6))
 (segment (start 152.4 78.58125) (end 154.78125 78.58125) (width 0.2) (layer "F.Cu") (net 6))
 (segment (start 155.947278 75.8825) (end 159.016 75.8825) (width 0.2) (layer "F.Cu") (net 6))
 (via (at 154.808904 77.020874) (size 0.6) (drill 0.3) (layers "F.Cu" "B.Cu") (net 6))
 (via (at 154.78125 78.58125) (size 0.6) (drill 0.3) (layers "F.Cu" "B.Cu") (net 6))
 (segment (start 154.78125 77.048528) (end 154.808904 77.020874) (width 0.2) (layer "B.Cu") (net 6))
 (segment (start 154.78125 78.58125) (end 154.78125 77.048528) (width 0.2) (layer "B.Cu") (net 6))
 (segment (start 174.256 81.3315) (end 174.256 80.9625) (width 0.2) (layer "F.Cu") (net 13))
 (segment (start 162.8775 92.71) (end 174.256 81.3315) (width 0.2) (layer "F.Cu") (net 13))
 (segment (start 143.8275 108.851) (end 174.256 78.4225) (width 0.2) (layer "F.Cu") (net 14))
 (segment (start 143.8275 111.76) (end 143.8275 108.851) (width 0.2) (layer "F.Cu") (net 14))
 (segment (start 171.45 76.2) (end 171.7675 75.8825) (width 0.2) (layer "F.Cu") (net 15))
 (segment (start 171.7675 75.8825) (end 174.256 75.8825) (width 0.2) (layer "F.Cu") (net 15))
 (segment (start 164.30625 110.33125) (end 164.30625 109.82) (width 0.2) (layer "F.Cu") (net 15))
 (segment (start 162.8775 111.76) (end 164.30625 110.33125) (width 0.2) (layer "F.Cu") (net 15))
 (via (at 171.45 76.2) (size 0.6) (drill 0.3) (layers "F.Cu" "B.Cu") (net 15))
 (via (at 164.30625 109.82) (size 0.6) (drill 0.3) (layers "F.Cu" "B.Cu") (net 15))
 (segment (start 164.30625 83.34375) (end 171.45 76.2) (width 0.2) (layer "B.Cu") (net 15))
 (segment (start 164.30625 109.82) (end 164.30625 83.34375) (width 0.2) (layer "B.Cu") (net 15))
 (segment (start 180.975 110.8075) (end 180.975 100.0125) (width 0.2) (layer "F.Cu") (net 5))
 (segment (start 178.59375 73.81875) (end 178.1175 73.3425) (width 0.2) (layer "F.Cu") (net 5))
 (segment (start 181.9275 111.76) (end 180.975 110.8075) (width 0.2) (layer "F.Cu") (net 5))
 (segment (start 178.1175 73.3425) (end 174.256 73.3425) (width 0.2) (layer "F.Cu") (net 5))
 (via (at 178.59375 73.81875) (size 0.6) (drill 0.3) (layers "F.Cu" "B.Cu") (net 5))
 (via (at 180.975 100.0125) (size 0.6) (drill 0.3) (layers "F.Cu" "B.Cu") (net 5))
 (segment (start 180.975 76.2) (end 178.59375 73.81875) (width 0.2) (layer "B.Cu") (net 5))
 (segment (start 180.975 100.0125) (end 180.975 76.2) (width 0.2) (layer "B.Cu") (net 5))
 (segment (start 178.6125 92.75) (end 178.6125 90.50625) (width 0.2) (layer "F.Cu") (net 7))
 (segment (start 169.493015 79.005515) (end 169.493015 76.199515) (width 0.2) (layer "F.Cu") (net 7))
 (segment (start 178.6125 90.50625) (end 174.255515 86.149265) (width 0.2) (layer "F.Cu") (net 7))
 (segment (start 169.493015 76.199515) (end 159.016 65.7225) (width 0.2) (layer "F.Cu") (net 7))
 (via (at 174.255515 86.149265) (size 0.6) (drill 0.3) (layers "F.Cu" "B.Cu") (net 7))
 (via (at 169.493015 79.005515) (size 0.6) (drill 0.3) (layers "F.Cu" "B.Cu") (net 7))
 (segment (start 169.493015 81.386765) (end 169.493015 79.005515) (width 0.2) (layer "B.Cu") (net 7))
 (segment (start 174.255515 86.149265) (end 169.493015 81.386765) (width 0.2) (layer "B.Cu") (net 7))
 (segment (start 176.2125 100.0125) (end 176.35 100.0125) (width 0.2) (layer "F.Cu") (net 8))
 (segment (start 176.35 100.0125) (end 178.6125 97.75) (width 0.2) (layer "F.Cu") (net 8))
 (segment (start 159.016 68.2625) (end 168.777485 78.023985) (width 0.2) (layer "F.Cu") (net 8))
 (segment (start 168.777485 78.023985) (end 168.777485 83.052485) (width 0.2) (layer "F.Cu") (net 8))
 (via (at 168.777485 83.052485) (size 0.6) (drill 0.3) (layers "F.Cu" "B.Cu") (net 8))
 (via (at 176.2125 100.0125) (size 0.6) (drill 0.3) (layers "F.Cu" "B.Cu") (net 8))
 (segment (start 176.2125 90.4875) (end 176.2125 100.0125) (width 0.2) (layer "B.Cu") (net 8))
 (segment (start 168.777485 83.052485) (end 176.2125 90.4875) (width 0.2) (layer "B.Cu") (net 8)))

